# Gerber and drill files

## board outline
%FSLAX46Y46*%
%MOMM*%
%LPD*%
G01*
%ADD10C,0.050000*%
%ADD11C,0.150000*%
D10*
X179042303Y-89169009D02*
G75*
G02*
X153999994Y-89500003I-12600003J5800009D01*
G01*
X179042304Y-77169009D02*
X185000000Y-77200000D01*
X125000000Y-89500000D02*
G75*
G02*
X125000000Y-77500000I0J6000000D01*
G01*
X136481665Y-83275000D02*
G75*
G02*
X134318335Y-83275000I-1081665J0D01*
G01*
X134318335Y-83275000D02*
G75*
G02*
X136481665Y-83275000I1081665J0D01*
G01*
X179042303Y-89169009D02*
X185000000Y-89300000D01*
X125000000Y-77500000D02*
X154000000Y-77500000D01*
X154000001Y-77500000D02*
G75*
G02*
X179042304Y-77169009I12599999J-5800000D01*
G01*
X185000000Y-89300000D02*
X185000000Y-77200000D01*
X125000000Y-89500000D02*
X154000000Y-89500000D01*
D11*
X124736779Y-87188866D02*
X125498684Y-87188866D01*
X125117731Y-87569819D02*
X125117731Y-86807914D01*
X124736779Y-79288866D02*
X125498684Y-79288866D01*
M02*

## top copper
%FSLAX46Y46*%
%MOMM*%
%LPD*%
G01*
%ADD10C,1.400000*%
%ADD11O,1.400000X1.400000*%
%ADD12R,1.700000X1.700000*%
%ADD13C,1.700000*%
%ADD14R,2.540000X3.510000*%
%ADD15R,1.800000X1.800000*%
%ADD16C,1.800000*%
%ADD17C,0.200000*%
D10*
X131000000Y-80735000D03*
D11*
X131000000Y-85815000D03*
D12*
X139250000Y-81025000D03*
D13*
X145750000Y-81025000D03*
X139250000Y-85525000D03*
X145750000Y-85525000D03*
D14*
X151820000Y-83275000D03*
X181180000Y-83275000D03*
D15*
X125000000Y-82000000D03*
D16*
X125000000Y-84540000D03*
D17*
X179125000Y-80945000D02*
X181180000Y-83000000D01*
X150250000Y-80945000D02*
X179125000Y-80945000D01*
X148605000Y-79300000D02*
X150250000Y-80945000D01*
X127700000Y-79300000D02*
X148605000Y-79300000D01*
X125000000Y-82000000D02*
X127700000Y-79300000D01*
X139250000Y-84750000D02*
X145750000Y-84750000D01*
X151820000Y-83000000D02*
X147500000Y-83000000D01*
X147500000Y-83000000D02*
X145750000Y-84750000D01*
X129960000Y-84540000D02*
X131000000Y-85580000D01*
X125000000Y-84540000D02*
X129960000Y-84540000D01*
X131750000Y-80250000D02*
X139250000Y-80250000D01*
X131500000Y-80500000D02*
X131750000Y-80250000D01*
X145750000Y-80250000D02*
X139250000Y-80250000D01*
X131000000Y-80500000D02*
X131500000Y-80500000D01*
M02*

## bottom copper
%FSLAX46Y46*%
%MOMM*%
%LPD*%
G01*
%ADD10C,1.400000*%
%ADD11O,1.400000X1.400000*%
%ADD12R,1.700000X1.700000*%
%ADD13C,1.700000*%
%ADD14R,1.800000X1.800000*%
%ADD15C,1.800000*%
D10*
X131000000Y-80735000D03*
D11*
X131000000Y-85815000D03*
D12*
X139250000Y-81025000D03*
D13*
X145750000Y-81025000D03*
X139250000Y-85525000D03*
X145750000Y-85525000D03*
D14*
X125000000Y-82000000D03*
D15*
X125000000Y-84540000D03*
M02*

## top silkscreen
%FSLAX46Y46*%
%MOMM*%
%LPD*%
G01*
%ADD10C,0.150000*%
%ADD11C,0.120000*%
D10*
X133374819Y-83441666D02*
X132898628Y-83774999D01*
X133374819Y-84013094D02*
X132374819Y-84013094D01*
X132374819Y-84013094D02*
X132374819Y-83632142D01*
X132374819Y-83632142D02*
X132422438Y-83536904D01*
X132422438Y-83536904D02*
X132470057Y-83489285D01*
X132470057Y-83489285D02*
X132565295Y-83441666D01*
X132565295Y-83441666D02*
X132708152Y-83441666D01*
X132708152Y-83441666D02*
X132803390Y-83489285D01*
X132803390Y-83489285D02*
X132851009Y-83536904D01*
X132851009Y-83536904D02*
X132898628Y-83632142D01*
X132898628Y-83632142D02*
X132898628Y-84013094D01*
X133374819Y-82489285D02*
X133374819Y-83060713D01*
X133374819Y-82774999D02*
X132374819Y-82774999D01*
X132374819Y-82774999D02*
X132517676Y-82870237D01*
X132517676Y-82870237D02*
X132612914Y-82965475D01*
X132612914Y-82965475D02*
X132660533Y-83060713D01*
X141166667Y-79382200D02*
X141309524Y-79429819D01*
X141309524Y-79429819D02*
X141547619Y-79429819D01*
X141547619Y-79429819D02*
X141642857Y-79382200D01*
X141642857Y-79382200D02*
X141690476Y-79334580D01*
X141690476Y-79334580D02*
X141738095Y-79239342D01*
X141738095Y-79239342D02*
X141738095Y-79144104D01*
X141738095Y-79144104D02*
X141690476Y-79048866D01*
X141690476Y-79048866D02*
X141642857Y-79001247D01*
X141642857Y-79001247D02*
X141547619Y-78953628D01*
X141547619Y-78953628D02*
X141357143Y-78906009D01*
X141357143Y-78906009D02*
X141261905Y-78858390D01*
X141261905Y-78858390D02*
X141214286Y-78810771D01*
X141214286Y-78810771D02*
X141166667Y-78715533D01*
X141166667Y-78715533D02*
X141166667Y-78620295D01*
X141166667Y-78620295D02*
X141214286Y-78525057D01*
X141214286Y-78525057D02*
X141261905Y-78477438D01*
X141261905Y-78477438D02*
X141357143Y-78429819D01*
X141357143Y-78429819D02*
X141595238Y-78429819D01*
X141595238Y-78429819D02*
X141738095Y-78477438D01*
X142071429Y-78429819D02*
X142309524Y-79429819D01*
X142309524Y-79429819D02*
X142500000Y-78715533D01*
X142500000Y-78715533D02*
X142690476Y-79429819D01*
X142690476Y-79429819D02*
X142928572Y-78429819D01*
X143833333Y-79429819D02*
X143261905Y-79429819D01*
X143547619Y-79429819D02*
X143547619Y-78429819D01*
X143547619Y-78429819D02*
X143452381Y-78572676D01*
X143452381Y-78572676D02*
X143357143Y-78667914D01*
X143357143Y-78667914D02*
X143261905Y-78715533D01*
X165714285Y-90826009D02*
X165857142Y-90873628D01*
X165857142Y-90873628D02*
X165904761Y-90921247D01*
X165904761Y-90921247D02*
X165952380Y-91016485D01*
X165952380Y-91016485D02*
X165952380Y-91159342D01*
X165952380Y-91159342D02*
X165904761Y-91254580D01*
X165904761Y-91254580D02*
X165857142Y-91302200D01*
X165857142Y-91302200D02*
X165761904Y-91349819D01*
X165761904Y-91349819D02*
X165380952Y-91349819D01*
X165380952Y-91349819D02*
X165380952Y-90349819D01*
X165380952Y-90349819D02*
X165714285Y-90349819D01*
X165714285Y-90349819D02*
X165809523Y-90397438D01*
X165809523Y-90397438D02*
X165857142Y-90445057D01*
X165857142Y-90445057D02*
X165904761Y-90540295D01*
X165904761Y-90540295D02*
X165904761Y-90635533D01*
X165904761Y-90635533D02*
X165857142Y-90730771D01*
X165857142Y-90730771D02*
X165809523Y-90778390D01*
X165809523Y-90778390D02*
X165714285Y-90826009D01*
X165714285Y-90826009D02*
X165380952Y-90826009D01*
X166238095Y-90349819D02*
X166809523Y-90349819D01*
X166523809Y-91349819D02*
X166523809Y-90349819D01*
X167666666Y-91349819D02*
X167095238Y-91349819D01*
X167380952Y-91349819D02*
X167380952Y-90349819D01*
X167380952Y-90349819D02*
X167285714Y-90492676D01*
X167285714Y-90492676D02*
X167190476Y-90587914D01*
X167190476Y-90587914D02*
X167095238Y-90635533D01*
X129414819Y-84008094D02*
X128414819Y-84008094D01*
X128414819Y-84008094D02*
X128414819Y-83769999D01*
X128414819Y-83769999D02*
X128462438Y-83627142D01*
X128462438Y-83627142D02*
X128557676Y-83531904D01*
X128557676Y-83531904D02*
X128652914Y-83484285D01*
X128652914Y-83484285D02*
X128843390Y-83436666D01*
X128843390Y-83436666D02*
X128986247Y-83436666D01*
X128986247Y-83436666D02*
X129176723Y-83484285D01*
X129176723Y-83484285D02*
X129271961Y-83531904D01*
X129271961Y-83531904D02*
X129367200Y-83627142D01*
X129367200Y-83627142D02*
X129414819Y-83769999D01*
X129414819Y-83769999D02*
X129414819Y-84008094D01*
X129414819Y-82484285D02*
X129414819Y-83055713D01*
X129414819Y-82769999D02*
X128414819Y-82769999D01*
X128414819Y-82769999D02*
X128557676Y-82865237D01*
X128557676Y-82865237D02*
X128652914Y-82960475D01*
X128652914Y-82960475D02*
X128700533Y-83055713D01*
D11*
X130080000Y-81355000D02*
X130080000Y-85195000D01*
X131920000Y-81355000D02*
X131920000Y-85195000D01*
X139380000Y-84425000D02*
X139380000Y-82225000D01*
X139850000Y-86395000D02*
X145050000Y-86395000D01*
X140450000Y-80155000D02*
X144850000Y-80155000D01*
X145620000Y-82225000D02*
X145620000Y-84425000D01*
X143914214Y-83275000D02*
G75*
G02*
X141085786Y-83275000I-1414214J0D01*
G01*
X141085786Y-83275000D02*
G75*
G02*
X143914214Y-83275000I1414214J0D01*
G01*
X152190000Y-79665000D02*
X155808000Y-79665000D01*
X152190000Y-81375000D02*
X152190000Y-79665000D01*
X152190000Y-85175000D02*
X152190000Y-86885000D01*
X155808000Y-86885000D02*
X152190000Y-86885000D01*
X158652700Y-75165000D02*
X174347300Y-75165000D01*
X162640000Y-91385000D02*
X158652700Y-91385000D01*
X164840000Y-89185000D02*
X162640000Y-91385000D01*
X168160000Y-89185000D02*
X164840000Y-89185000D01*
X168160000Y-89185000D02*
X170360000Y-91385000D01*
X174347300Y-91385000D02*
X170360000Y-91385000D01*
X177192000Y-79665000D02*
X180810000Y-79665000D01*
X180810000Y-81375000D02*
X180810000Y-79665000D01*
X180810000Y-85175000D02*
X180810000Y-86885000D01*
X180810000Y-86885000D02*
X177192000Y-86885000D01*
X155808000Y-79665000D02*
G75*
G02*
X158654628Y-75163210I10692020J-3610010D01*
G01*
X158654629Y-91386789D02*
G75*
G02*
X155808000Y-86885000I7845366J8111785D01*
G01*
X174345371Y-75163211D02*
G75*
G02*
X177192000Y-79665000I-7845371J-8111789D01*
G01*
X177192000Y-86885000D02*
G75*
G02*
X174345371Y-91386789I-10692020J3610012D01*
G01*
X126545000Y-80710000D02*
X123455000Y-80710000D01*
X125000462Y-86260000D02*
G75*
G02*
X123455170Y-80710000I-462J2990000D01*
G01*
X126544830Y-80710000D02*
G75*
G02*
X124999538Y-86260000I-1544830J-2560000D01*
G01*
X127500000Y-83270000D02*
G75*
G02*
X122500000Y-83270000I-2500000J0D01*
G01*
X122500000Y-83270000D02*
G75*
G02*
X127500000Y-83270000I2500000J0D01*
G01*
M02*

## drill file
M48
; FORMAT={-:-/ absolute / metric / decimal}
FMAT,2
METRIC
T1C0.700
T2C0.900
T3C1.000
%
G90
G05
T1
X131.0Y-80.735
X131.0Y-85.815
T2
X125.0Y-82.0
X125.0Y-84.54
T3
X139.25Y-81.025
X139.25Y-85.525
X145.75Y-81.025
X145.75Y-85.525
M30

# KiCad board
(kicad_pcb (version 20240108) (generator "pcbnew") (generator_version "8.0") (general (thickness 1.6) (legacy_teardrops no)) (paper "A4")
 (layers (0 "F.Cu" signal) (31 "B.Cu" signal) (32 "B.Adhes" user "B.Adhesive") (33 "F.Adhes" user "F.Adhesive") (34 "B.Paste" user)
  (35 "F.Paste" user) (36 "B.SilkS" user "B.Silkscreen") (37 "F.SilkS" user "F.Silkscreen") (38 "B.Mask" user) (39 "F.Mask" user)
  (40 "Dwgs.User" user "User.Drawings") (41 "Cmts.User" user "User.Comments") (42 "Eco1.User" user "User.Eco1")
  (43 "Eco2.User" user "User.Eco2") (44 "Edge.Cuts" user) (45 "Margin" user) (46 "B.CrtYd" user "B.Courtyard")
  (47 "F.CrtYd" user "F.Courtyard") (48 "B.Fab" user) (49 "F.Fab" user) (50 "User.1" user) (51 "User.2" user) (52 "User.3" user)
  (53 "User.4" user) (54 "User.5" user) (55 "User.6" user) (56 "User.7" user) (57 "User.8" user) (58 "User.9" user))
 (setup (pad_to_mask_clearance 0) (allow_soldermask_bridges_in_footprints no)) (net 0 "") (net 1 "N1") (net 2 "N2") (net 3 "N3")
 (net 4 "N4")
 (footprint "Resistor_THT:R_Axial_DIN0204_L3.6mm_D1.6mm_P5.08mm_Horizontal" (layer "F.Cu") (at 131 80.735 -90)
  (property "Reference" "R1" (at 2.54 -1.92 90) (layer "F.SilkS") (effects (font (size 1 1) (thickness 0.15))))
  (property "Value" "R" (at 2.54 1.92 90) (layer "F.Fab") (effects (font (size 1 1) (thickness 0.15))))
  (fp_line (start 0.62 0.92) (end 4.46 0.92) (stroke (width 0.12) (type solid)) (layer "F.SilkS"))
  (fp_line (start 0.62 -0.92) (end 4.46 -0.92) (stroke (width 0.12) (type solid)) (layer "F.SilkS"))
  (pad "1" thru_hole circle (at 0 0 270) (size 1.4 1.4) (drill 0.7) (layers "*.Cu" "*.Mask") (remove_unused_layers no) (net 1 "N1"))
  (pad "2" thru_hole oval (at 5.08 0 270) (size 1.4 1.4) (drill 0.7) (layers "*.Cu" "*.Mask") (remove_unused_layers no) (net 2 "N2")))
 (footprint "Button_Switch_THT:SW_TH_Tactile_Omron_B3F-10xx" (layer "F.Cu") (at 139.25 81.025)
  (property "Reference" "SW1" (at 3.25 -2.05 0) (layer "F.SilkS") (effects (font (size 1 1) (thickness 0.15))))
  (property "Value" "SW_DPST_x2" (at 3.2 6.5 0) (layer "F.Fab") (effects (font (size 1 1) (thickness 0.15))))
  (fp_line (start 0.13 3.4) (end 0.13 1.2) (stroke (width 0.12) (type solid)) (layer "F.SilkS"))
  (fp_line (start 0.6 5.37) (end 5.8 5.37) (stroke (width 0.12) (type solid)) (layer "F.SilkS"))
  (fp_line (start 1.2 -0.87) (end 5.6 -0.87) (stroke (width 0.12) (type solid)) (layer "F.SilkS"))
  (fp_line (start 6.37 1.2) (end 6.37 3.4) (stroke (width 0.12) (type solid)) (layer "F.SilkS"))
  (fp_circle (center 3.25 2.25) (end 4.25 3.25) (stroke (width 0.12) (type solid)) (fill none) (layer "F.SilkS"))
  (pad "1" thru_hole rect (at 0 0) (size 1.7 1.7) (drill 1) (layers "*.Cu" "*.Mask") (remove_unused_layers no) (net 1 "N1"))
  (pad "1" thru_hole circle (at 6.5 0) (size 1.7 1.7) (drill 1) (layers "*.Cu" "*.Mask") (remove_unused_layers no) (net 1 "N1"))
  (pad "2" thru_hole circle (at 0 4.5) (size 1.7 1.7) (drill 1) (layers "*.Cu" "*.Mask") (remove_unused_layers no) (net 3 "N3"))
  (pad "2" thru_hole circle (at 6.5 4.5) (size 1.7 1.7) (drill 1) (layers "*.Cu" "*.Mask") (remove_unused_layers no) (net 3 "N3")))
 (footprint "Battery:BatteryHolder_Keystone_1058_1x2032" (layer "F.Cu") (at 166.5 83.275)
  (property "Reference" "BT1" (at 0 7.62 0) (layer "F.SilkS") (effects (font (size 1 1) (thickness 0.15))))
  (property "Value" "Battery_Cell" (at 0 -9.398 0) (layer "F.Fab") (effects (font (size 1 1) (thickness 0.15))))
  (fp_line (start -14.31 -3.61) (end -10.692 -3.61) (stroke (width 0.12) (type solid)) (layer "F.SilkS"))
  (fp_line (start -14.31 -1.9) (end -14.31 -3.61) (stroke (width 0.12) (type solid)) (layer "F.SilkS"))
  (fp_line (start -14.31 1.9) (end -14.31 3.61) (stroke (width 0.12) (type solid)) (layer "F.SilkS"))
  (fp_line (start -10.692 3.61) (end -14.31 3.61) (stroke (width 0.12) (type solid)) (layer "F.SilkS"))
  (fp_line (start -7.8473 -8.11) (end 7.8473 -8.11) (stroke (width 0.12) (type solid)) (layer "F.SilkS"))
  (fp_line (start -3.86 8.11) (end -7.8473 8.11) (stroke (width 0.12) (type solid)) (layer "F.SilkS"))
  (fp_line (start -1.66 5.91) (end -3.86 8.11) (stroke (width 0.12) (type solid)) (layer "F.SilkS"))
  (fp_line (start 1.66 5.91) (end -1.66 5.91) (stroke (width 0.12) (type solid)) (layer "F.SilkS"))
  (fp_line (start 1.66 5.91) (end 3.86 8.11) (stroke (width 0.12) (type solid)) (layer "F.SilkS"))
  (fp_line (start 7.8473 8.11) (end 3.86 8.11) (stroke (width 0.12) (type solid)) (layer "F.SilkS"))
  (fp_line (start 10.692 -3.61) (end 14.31 -3.61) (stroke (width 0.12) (type solid)) (layer "F.SilkS"))
  (fp_line (start 14.31 -1.9) (end 14.31 -3.61) (stroke (width 0.12) (type solid)) (layer "F.SilkS"))
  (fp_line (start 14.31 1.9) (end 14.31 3.61) (stroke (width 0.12) (type solid)) (layer "F.SilkS"))
  (fp_line (start 14.31 3.61) (end 10.692 3.61) (stroke (width 0.12) (type solid)) (layer "F.SilkS"))
  (fp_arc (start -10.692 -3.61) (mid -9.538084 -6.031244) (end -7.845371 -8.111789) (stroke (width 0.12) (type solid)) (layer "F.SilkS"))
  (fp_arc (start -7.845371 8.111789) (mid -9.538085 6.031244) (end -10.692 3.61) (stroke (width 0.12) (type solid)) (layer "F.SilkS"))
  (fp_arc (start 7.845371 -8.111789) (mid 9.538085 -6.031244) (end 10.692 -3.61) (stroke (width 0.12) (type solid)) (layer "F.SilkS"))
  (fp_arc (start 10.692 3.61) (mid 9.538084 6.031244) (end 7.845371 8.111789) (stroke (width 0.12) (type solid)) (layer "F.SilkS"))
  (pad "1" smd rect (at -14.68 0) (size 2.54 3.51) (layers "F.Cu" "F.Paste" "F.Mask") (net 3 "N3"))
  (pad "2" smd rect (at 14.68 0) (size 2.54 3.51) (layers "F.Cu" "F.Paste" "F.Mask") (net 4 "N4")))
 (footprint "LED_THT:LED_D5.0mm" (layer "F.Cu") (at 125 82 -90)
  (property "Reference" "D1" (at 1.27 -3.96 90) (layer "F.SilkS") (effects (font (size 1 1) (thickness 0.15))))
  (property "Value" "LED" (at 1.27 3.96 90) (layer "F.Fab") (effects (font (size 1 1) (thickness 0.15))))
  (fp_line (start -1.29 -1.545) (end -1.29 1.545) (stroke (width 0.12) (type solid)) (layer "F.SilkS"))
  (fp_arc (start 4.26 -0.000462) (mid 2.072002 2.880433) (end -1.29 1.54483) (stroke (width 0.12) (type solid)) (layer "F.SilkS"))
  (fp_arc (start -1.29 -1.54483) (mid 2.072002 -2.880433) (end 4.26 0.000462) (stroke (width 0.12) (type solid)) (layer "F.SilkS"))
  (fp_circle (center 1.27 0) (end 3.77 0) (stroke (width 0.12) (type solid)) (fill none) (layer "F.SilkS"))
  (pad "1" thru_hole rect (at 0 0 270) (size 1.8 1.8) (drill 0.9) (layers "*.Cu" "*.Mask") (remove_unused_layers no) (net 4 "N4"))
  (pad "2" thru_hole circle (at 2.54 0 270) (size 1.8 1.8) (drill 0.9) (layers "*.Cu" "*.Mask") (remove_unused_layers no) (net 2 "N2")))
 (gr_arc (start 179.042303 89.169009) (mid 166.625623 97.238629) (end 154 89.5) (stroke (width 0.05) (type default)) (layer "Edge.Cuts"))
 (gr_line (start 179.042304 77.169009) (end 185 77.2) (stroke (width 0.05) (type default)) (layer "Edge.Cuts"))
 (gr_arc (start 125 89.5) (mid 119 83.5) (end 125 77.5) (stroke (width 0.05) (type default)) (layer "Edge.Cuts"))
 (gr_circle (center 135.4 83.275) (end 136.3 83.875) (stroke (width 0.05) (type default)) (fill none) (layer "Edge.Cuts"))
 (gr_line (start 179.042303 89.169009) (end 185 89.3) (stroke (width 0.05) (type default)) (layer "Edge.Cuts"))
 (gr_line (start 125 77.5) (end 154 77.5) (stroke (width 0.05) (type default)) (layer "Edge.Cuts"))
 (gr_arc (start 154.000001 77.5) (mid 166.416681 69.43038) (end 179.042304 77.169009) (stroke (width 0.05) (type default))
  (layer "Edge.Cuts"))
 (gr_line (start 185 89.3) (end 185 77.2) (stroke (width 0.05) (type default)) (layer "Edge.Cuts"))
 (gr_line (start 125 89.5) (end 154 89.5) (stroke (width 0.05) (type default)) (layer "Edge.Cuts"))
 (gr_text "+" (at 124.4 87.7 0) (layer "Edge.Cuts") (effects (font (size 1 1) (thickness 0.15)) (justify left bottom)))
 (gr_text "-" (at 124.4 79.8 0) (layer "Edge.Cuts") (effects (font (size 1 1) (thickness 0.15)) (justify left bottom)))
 (segment (start 179.125 80.945) (end 181.18 83) (width 0.2) (layer "F.Cu") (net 4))
 (segment (start 150.25 80.945) (end 179.125 80.945) (width 0.2) (layer "F.Cu") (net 4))
 (segment (start 148.605 79.3) (end 150.25 80.945) (width 0.2) (layer "F.Cu") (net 4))
 (segment (start 127.7 79.3) (end 148.605 79.3) (width 0.2) (layer "F.Cu") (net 4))
 (segment (start 125 82) (end 127.7 79.3) (width 0.2) (layer "F.Cu") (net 4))
 (segment (start 139.25 84.75) (end 145.75 84.75) (width 0.2) (layer "F.Cu") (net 3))
 (segment (start 151.82 83) (end 147.5 83) (width 0.2) (layer "F.Cu") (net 3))
 (segment (start 147.5 83) (end 145.75 84.75) (width 0.2) (layer "F.Cu") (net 3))
 (segment (start 129.96 84.54) (end 131 85.58) (width 0.2) (layer "F.Cu") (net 2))
 (segment (start 125 84.54) (end 129.96 84.54) (width 0.2) (layer "F.Cu") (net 2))
 (segment (start 131.75 80.25) (end 139.25 80.25) (width 0.2) (layer "F.Cu") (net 1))
 (segment (start 131.5 80.5) (end 131.75 80.25) (width 0.2) (layer "F.Cu") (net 1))
 (segment (start 145.75 80.25) (end 139.25 80.25) (width 0.2) (layer "F.Cu") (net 1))
 (segment (start 131 80.5) (end 131.5 80.5) (width 0.2) (layer "F.Cu") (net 1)))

